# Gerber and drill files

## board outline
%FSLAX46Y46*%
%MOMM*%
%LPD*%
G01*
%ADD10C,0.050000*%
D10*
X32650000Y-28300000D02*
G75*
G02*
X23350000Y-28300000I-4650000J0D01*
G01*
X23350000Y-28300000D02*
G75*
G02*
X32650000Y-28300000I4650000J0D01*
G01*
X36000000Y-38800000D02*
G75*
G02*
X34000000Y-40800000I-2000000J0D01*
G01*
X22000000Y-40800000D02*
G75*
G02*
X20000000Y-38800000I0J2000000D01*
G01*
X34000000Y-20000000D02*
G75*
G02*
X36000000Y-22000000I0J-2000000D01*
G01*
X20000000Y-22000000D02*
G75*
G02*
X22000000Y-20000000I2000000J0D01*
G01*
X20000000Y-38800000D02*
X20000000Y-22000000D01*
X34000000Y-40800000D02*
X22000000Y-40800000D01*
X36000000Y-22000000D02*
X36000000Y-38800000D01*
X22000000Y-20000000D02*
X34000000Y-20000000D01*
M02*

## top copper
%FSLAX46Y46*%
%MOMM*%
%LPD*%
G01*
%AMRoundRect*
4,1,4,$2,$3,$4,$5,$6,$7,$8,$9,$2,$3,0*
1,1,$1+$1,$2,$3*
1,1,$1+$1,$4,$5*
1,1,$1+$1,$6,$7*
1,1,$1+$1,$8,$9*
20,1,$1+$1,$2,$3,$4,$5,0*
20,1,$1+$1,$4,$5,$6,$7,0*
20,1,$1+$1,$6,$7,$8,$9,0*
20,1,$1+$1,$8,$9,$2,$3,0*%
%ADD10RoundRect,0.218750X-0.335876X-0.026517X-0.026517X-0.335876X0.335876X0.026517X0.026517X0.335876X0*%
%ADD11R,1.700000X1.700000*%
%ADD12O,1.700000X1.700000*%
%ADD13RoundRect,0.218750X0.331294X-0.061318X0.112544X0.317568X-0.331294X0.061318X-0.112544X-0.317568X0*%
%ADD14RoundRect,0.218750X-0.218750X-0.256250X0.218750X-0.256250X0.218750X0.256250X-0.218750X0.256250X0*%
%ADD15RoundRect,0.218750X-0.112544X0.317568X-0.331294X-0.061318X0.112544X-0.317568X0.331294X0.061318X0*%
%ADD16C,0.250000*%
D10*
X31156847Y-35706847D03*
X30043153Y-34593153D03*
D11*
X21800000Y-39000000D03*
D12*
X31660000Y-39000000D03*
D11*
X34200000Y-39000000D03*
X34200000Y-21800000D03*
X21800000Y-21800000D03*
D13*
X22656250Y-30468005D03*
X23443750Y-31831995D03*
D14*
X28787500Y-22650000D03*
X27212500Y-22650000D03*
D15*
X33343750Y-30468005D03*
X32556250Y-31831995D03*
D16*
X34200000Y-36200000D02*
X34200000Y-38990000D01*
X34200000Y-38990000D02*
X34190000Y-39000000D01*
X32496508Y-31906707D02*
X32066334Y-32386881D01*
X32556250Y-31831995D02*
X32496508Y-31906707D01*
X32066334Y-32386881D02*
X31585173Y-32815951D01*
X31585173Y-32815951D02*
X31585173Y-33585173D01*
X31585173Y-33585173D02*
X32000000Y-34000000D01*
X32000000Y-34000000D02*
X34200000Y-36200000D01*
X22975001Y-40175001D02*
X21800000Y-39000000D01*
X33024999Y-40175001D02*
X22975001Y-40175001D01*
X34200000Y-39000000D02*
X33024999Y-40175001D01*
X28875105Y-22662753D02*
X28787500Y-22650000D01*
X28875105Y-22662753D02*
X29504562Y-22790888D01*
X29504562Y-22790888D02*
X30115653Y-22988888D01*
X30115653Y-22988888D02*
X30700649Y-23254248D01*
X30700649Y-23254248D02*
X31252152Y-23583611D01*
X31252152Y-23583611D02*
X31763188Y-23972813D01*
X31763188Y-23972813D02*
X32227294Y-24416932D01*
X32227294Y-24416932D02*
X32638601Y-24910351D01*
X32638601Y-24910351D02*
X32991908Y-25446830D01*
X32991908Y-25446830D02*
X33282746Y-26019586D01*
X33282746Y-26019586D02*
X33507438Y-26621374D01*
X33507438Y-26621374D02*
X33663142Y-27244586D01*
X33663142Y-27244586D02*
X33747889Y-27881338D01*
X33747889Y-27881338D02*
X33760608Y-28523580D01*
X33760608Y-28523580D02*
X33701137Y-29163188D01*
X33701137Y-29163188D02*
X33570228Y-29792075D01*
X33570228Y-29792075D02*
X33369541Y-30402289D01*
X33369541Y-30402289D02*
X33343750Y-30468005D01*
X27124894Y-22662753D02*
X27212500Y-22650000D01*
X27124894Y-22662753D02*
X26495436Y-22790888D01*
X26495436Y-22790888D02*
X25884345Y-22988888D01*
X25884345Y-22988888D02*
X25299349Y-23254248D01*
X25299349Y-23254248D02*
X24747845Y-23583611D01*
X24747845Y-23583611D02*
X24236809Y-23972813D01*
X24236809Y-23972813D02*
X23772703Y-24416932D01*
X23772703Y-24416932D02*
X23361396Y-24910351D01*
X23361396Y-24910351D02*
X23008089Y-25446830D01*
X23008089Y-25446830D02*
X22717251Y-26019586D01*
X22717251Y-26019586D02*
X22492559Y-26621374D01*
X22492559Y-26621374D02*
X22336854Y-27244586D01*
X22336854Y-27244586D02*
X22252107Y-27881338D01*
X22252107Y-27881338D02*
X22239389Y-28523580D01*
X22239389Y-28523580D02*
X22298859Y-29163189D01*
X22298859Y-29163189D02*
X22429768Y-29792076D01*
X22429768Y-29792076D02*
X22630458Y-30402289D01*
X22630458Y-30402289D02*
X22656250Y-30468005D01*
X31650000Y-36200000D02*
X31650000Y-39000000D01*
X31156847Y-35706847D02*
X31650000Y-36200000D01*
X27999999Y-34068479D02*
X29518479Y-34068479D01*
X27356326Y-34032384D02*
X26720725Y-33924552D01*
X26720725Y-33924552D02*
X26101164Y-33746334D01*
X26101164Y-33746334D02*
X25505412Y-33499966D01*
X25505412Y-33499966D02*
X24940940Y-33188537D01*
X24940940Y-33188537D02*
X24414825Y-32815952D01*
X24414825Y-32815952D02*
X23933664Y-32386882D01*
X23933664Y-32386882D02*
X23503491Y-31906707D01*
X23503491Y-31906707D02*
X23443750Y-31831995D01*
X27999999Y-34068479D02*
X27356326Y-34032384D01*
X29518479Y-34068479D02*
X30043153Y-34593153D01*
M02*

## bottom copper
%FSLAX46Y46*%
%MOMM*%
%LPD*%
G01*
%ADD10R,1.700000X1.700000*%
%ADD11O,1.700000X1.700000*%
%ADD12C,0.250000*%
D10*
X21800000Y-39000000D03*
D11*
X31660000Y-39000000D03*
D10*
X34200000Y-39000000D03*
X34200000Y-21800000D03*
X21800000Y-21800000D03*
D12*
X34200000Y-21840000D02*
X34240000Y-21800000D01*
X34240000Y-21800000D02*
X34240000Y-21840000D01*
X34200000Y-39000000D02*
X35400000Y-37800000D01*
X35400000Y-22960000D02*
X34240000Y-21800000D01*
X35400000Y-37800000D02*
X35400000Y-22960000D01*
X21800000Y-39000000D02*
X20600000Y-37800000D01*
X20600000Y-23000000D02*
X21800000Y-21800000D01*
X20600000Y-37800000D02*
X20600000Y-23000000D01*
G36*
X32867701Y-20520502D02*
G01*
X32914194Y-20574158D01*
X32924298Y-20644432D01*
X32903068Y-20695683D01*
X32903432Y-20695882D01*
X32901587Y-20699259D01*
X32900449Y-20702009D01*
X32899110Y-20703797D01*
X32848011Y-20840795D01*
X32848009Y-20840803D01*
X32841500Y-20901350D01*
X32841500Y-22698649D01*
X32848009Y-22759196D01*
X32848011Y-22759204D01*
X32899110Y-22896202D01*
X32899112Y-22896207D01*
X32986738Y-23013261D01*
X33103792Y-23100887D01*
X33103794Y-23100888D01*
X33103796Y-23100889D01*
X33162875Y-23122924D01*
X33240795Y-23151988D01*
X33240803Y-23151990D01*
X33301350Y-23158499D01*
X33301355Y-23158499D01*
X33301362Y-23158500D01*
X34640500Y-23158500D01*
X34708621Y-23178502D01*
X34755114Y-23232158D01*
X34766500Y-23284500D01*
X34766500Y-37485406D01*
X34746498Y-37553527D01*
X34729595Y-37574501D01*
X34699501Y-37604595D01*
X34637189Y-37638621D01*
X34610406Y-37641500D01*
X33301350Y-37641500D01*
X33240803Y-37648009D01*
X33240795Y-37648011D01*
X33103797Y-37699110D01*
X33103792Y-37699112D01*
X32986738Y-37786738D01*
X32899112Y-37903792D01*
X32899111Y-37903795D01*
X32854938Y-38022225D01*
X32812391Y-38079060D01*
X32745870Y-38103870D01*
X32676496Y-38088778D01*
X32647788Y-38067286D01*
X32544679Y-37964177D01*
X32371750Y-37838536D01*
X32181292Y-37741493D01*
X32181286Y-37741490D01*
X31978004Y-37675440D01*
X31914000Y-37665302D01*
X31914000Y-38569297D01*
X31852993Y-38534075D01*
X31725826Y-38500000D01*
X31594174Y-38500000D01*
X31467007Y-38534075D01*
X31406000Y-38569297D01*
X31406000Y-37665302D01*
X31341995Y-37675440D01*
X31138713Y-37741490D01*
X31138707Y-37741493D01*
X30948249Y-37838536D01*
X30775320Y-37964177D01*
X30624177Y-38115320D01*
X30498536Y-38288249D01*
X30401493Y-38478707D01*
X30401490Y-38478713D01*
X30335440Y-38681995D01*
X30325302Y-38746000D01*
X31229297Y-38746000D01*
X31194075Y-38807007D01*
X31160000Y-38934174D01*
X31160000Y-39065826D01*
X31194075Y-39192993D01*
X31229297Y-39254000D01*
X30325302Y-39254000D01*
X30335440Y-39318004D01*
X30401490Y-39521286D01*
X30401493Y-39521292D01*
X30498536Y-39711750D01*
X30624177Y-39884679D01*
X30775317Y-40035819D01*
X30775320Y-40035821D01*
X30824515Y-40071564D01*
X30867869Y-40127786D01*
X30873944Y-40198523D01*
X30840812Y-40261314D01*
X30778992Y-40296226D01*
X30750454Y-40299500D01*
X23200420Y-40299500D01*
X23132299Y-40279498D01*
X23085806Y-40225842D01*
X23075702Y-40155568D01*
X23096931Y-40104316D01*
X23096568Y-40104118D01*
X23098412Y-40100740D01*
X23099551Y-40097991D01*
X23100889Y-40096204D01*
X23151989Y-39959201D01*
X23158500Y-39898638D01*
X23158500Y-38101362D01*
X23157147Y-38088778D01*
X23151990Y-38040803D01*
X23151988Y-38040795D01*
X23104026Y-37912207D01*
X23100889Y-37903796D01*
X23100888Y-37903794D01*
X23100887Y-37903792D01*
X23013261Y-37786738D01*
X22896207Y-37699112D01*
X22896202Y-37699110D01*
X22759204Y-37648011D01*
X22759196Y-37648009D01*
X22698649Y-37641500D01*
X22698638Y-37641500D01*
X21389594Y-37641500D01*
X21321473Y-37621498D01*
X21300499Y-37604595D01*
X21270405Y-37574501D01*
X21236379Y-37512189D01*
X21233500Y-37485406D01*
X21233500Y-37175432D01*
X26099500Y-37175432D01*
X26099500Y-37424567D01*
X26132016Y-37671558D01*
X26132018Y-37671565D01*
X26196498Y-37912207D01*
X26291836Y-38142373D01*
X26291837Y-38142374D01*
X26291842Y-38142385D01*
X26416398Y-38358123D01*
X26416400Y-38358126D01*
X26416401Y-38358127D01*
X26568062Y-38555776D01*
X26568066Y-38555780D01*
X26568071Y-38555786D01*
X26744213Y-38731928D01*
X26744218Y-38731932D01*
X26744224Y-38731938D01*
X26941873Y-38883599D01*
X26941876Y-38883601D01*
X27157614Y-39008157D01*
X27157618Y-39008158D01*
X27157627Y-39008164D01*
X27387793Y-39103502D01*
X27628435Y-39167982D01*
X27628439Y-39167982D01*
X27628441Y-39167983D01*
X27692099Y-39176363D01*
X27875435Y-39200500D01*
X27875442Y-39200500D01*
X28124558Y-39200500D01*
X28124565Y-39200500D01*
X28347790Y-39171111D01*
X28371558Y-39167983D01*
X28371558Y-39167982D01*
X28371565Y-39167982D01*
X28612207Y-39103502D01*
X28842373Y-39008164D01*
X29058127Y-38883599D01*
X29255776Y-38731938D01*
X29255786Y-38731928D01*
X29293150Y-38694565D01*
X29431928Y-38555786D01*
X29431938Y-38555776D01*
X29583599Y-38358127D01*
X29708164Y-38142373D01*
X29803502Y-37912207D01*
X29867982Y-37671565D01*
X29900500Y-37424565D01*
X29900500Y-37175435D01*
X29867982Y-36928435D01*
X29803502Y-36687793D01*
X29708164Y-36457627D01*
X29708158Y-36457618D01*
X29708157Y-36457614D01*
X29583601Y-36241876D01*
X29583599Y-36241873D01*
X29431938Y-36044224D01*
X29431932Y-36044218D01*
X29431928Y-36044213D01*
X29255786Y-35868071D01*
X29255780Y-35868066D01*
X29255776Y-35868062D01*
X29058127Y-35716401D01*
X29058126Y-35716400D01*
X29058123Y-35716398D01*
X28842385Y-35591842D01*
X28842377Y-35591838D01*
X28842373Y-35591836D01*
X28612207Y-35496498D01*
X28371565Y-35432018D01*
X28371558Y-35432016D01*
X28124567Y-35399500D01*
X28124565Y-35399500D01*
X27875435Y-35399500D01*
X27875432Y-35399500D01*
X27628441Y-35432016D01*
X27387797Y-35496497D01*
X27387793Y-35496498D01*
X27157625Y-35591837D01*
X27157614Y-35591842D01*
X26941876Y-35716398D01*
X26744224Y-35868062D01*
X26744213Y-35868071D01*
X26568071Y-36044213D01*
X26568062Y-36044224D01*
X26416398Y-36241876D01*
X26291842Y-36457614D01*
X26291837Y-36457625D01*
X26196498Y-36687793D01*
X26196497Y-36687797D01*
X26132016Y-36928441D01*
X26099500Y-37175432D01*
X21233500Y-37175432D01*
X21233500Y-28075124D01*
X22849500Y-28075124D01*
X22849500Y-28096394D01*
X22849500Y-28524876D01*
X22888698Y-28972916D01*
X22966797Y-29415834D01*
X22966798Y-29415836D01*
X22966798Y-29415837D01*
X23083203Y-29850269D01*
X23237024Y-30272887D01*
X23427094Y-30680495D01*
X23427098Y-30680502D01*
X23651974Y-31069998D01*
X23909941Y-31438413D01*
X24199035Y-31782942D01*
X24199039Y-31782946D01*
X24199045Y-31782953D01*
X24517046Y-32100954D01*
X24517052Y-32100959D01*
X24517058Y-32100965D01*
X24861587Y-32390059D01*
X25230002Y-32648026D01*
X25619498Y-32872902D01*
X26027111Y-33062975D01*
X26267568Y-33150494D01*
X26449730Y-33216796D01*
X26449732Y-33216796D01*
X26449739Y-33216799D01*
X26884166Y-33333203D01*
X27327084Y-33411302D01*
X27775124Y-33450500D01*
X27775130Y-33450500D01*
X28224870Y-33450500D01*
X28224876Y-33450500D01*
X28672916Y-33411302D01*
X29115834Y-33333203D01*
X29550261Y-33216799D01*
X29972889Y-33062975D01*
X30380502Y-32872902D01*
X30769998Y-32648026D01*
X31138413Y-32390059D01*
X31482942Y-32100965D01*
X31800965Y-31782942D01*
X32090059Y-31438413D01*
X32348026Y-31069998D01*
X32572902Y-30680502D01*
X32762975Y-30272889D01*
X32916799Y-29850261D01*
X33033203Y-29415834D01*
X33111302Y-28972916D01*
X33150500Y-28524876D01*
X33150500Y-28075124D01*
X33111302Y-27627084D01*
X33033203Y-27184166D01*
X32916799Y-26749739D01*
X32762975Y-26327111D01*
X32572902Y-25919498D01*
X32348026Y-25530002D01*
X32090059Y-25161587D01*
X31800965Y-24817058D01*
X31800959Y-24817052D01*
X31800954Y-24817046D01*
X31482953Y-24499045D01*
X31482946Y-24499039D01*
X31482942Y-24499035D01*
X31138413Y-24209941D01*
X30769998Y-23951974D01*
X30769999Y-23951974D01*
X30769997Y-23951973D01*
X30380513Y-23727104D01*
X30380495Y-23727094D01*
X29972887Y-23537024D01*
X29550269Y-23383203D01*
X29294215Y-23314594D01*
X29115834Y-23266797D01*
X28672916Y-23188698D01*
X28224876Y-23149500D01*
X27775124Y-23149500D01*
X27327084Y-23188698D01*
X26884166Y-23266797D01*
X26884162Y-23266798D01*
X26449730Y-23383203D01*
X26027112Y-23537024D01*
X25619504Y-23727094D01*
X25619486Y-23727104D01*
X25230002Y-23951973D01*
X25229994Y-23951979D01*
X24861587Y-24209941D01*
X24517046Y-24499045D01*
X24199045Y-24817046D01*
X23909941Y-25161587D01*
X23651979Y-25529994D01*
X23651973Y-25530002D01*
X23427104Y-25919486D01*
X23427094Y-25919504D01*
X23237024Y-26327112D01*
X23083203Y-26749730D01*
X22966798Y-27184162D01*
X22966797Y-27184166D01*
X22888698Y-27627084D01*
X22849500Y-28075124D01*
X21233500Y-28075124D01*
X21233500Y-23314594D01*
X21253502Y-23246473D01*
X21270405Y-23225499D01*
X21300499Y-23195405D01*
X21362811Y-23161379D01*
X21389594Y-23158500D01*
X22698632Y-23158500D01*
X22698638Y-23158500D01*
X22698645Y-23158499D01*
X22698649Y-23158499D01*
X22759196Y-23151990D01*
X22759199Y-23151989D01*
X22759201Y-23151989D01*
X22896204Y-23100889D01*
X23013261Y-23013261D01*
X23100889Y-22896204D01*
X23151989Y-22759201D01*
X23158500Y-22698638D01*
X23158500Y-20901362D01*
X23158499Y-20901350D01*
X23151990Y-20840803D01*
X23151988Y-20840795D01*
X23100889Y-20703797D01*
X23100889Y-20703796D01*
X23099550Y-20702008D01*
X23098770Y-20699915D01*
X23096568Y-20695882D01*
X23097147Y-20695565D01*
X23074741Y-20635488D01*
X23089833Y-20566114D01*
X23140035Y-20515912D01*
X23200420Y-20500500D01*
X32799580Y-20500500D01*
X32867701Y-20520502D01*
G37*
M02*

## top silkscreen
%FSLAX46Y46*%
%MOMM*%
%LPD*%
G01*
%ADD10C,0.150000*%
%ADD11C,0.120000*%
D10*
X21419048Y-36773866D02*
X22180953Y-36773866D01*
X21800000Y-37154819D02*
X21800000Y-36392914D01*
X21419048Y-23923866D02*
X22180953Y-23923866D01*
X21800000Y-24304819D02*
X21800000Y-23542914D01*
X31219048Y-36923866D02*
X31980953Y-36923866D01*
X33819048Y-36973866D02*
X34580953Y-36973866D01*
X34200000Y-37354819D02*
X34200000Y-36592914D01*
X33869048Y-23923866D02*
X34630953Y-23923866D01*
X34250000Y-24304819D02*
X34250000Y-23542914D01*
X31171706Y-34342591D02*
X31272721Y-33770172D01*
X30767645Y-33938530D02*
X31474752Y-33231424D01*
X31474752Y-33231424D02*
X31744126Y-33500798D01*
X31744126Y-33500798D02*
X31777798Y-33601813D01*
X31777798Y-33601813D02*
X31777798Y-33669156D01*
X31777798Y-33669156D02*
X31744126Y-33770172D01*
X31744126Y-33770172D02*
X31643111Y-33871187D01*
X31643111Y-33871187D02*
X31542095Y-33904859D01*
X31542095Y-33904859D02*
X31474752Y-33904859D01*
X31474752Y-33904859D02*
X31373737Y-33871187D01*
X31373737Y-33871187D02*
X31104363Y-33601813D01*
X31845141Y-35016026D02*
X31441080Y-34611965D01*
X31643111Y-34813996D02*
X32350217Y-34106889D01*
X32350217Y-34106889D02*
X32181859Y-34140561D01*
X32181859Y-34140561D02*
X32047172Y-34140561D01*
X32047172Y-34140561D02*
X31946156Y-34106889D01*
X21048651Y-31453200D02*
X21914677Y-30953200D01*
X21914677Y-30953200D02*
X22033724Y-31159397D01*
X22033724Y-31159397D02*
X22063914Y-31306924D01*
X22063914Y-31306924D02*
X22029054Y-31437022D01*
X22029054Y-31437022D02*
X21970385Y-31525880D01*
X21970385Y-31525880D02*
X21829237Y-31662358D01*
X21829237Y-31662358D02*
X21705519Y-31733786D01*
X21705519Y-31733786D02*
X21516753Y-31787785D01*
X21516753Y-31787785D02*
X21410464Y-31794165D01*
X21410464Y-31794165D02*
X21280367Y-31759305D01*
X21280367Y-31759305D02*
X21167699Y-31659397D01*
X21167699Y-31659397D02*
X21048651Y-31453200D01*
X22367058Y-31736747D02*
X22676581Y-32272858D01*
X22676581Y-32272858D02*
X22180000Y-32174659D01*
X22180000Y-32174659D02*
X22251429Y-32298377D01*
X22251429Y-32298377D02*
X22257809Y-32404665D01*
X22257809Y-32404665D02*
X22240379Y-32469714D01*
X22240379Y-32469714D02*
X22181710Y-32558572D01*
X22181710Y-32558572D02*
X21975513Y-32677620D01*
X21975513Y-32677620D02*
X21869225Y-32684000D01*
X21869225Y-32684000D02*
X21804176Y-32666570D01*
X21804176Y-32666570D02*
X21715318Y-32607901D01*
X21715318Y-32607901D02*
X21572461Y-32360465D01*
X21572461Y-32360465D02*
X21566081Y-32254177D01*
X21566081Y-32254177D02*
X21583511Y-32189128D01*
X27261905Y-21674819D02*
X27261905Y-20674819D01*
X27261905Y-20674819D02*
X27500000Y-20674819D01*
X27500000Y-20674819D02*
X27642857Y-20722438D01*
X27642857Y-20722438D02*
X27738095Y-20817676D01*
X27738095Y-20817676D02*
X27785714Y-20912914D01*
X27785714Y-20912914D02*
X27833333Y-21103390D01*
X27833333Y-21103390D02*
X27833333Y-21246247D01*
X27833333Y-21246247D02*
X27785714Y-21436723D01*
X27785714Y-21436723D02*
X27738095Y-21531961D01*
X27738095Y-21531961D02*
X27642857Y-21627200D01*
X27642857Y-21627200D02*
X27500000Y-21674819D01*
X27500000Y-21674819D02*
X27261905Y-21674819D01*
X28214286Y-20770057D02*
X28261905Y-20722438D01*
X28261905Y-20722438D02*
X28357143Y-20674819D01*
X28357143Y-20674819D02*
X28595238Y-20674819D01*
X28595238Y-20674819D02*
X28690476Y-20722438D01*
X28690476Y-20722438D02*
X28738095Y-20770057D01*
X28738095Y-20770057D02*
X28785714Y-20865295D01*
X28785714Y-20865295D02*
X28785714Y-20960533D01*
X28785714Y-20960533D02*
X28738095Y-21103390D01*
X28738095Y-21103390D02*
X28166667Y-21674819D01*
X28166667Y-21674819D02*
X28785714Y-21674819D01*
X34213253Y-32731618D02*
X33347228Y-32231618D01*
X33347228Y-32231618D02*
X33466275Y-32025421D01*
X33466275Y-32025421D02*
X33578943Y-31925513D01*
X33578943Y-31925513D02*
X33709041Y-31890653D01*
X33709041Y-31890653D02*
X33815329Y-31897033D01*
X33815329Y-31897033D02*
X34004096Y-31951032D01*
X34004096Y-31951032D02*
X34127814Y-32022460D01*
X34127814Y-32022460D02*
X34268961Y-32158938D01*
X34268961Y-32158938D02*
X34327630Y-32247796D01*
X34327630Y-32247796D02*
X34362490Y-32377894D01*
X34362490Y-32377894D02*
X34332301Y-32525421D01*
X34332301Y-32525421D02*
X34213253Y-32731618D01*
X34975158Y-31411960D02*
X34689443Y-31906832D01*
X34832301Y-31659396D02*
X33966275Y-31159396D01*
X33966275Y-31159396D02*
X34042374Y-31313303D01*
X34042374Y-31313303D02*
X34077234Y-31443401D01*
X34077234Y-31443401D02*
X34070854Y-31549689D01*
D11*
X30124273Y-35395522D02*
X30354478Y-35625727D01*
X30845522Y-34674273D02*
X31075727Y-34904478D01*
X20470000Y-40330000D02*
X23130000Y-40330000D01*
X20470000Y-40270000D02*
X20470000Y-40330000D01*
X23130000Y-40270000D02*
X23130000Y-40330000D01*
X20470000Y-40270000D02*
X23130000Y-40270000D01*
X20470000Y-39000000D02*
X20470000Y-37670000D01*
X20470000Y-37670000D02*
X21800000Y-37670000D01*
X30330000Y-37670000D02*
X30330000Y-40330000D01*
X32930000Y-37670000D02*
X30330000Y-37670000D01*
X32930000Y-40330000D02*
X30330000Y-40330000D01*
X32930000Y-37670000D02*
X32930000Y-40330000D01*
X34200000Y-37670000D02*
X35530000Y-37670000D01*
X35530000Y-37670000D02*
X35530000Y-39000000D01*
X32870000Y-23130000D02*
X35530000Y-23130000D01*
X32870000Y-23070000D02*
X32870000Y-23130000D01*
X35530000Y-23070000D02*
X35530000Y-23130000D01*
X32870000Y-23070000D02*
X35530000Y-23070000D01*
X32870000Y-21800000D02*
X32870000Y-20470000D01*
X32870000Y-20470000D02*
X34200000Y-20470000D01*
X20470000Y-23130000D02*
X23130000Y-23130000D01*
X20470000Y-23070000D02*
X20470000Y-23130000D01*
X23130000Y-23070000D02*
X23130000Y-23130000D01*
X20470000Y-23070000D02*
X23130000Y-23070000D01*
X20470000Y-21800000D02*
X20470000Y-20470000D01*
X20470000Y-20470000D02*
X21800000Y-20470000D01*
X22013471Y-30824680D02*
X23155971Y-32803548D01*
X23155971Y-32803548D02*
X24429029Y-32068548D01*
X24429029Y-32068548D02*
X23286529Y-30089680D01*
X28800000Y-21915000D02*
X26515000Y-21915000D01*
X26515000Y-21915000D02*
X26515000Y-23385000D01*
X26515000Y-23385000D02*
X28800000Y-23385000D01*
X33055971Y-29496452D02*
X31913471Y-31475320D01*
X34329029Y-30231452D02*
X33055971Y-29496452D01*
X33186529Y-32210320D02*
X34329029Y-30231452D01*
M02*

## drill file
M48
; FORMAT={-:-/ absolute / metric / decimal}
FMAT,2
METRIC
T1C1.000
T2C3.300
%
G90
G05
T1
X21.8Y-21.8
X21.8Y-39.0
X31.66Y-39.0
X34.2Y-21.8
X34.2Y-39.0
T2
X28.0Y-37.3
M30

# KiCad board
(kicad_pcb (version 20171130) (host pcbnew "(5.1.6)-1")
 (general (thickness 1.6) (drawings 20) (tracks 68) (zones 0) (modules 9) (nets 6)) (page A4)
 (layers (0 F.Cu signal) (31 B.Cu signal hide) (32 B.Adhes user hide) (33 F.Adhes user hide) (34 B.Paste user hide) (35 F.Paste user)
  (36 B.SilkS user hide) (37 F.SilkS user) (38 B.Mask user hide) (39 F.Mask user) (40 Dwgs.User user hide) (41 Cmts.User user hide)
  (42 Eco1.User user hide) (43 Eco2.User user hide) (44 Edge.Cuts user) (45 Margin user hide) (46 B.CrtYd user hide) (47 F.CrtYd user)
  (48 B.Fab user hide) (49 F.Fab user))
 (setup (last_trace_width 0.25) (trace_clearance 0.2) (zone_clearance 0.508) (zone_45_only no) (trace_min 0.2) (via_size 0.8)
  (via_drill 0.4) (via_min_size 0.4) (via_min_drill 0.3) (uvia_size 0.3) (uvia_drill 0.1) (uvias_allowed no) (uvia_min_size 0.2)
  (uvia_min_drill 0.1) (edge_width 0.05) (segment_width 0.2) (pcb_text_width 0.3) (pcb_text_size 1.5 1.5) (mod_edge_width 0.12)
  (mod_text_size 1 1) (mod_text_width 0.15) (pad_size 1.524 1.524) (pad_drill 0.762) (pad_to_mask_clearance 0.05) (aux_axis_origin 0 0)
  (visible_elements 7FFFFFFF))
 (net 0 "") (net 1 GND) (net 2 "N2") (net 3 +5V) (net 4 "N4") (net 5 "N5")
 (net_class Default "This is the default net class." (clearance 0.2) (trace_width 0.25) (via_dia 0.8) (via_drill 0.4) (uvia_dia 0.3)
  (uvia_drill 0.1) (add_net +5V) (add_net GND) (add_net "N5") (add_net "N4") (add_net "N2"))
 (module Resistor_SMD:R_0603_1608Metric (layer F.Cu) (at 30.6 35.15 315)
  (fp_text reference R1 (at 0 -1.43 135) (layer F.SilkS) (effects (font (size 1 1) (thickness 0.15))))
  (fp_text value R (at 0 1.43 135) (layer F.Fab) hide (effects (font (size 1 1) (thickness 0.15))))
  (fp_line (start -0.162779 0.51) (end 0.162779 0.51) (layer F.SilkS) (width 0.12))
  (fp_line (start -0.162779 -0.51) (end 0.162779 -0.51) (layer F.SilkS) (width 0.12))
  (pad 2 smd roundrect (at 0.7875 0 315) (size 0.875 0.95) (layers F.Cu F.Paste F.Mask) (roundrect_rratio 0.25) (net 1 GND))
  (pad 1 smd roundrect (at -0.7875 0 315) (size 0.875 0.95) (layers F.Cu F.Paste F.Mask) (roundrect_rratio 0.25) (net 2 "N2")))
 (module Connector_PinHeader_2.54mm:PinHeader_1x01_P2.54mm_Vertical (layer F.Cu) (at 21.8 39)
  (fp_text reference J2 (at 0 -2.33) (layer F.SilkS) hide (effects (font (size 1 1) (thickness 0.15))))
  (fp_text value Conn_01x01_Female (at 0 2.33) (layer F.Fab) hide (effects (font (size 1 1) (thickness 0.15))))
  (fp_line (start -1.33 1.33) (end 1.33 1.33) (layer F.SilkS) (width 0.12))
  (fp_line (start -1.33 1.27) (end -1.33 1.33) (layer F.SilkS) (width 0.12))
  (fp_line (start 1.33 1.27) (end 1.33 1.33) (layer F.SilkS) (width 0.12))
  (fp_line (start -1.33 1.27) (end 1.33 1.27) (layer F.SilkS) (width 0.12))
  (fp_line (start -1.33 0) (end -1.33 -1.33) (layer F.SilkS) (width 0.12))
  (fp_line (start -1.33 -1.33) (end 0 -1.33) (layer F.SilkS) (width 0.12))
  (pad 1 thru_hole rect (at 0 0) (size 1.7 1.7) (drill 1) (layers *.Cu *.Mask) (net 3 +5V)))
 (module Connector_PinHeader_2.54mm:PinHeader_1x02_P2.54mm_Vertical (layer F.Cu) (at 34.2 39 270)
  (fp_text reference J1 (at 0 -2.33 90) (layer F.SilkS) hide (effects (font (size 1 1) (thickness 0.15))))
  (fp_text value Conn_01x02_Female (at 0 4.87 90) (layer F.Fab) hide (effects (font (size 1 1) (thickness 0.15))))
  (fp_line (start -1.33 3.87) (end 1.33 3.87) (layer F.SilkS) (width 0.12))
  (fp_line (start -1.33 1.27) (end -1.33 3.87) (layer F.SilkS) (width 0.12))
  (fp_line (start 1.33 1.27) (end 1.33 3.87) (layer F.SilkS) (width 0.12))
  (fp_line (start -1.33 1.27) (end 1.33 1.27) (layer F.SilkS) (width 0.12))
  (fp_line (start -1.33 0) (end -1.33 -1.33) (layer F.SilkS) (width 0.12))
  (fp_line (start -1.33 -1.33) (end 0 -1.33) (layer F.SilkS) (width 0.12))
  (pad 2 thru_hole oval (at 0 2.54 270) (size 1.7 1.7) (drill 1) (layers *.Cu *.Mask) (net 1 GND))
  (pad 1 thru_hole rect (at 0 0 270) (size 1.7 1.7) (drill 1) (layers *.Cu *.Mask) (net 3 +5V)))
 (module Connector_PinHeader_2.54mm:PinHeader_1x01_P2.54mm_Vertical (layer F.Cu) (at 34.2 21.8)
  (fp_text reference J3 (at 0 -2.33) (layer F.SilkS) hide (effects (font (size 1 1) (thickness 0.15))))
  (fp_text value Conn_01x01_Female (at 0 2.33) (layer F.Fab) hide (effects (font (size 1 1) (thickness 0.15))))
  (fp_line (start -1.33 1.33) (end 1.33 1.33) (layer F.SilkS) (width 0.12))
  (fp_line (start -1.33 1.27) (end -1.33 1.33) (layer F.SilkS) (width 0.12))
  (fp_line (start 1.33 1.27) (end 1.33 1.33) (layer F.SilkS) (width 0.12))
  (fp_line (start -1.33 1.27) (end 1.33 1.27) (layer F.SilkS) (width 0.12))
  (fp_line (start -1.33 0) (end -1.33 -1.33) (layer F.SilkS) (width 0.12))
  (fp_line (start -1.33 -1.33) (end 0 -1.33) (layer F.SilkS) (width 0.12))
  (pad 1 thru_hole rect (at 0 0) (size 1.7 1.7) (drill 1) (layers *.Cu *.Mask) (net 3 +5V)))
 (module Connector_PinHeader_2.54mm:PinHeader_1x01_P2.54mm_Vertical (layer F.Cu) (at 21.8 21.8)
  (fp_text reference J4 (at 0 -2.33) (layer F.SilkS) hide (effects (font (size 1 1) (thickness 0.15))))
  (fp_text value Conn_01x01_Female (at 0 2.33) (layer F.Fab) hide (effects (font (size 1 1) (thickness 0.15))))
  (fp_line (start -1.33 1.33) (end 1.33 1.33) (layer F.SilkS) (width 0.12))
  (fp_line (start -1.33 1.27) (end -1.33 1.33) (layer F.SilkS) (width 0.12))
  (fp_line (start 1.33 1.27) (end 1.33 1.33) (layer F.SilkS) (width 0.12))
  (fp_line (start -1.33 1.27) (end 1.33 1.27) (layer F.SilkS) (width 0.12))
  (fp_line (start -1.33 0) (end -1.33 -1.33) (layer F.SilkS) (width 0.12))
  (fp_line (start -1.33 -1.33) (end 0 -1.33) (layer F.SilkS) (width 0.12))
  (pad 1 thru_hole rect (at 0 0) (size 1.7 1.7) (drill 1) (layers *.Cu *.Mask) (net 3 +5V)))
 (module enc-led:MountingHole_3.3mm (layer F.Cu) (at 28 37.3)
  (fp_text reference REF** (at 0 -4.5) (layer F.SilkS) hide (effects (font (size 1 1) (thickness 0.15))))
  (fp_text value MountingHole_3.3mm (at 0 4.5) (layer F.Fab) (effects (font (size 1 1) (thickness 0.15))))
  (pad "" np_thru_hole circle (at 0 0) (size 3.3 3.3) (drill 3.3) (layers *.Cu *.Mask)))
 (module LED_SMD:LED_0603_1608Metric (layer F.Cu) (at 23.05 31.15 120)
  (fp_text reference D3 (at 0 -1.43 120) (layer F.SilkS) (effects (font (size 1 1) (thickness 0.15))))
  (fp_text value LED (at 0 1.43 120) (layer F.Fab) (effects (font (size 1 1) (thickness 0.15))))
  (fp_line (start 0.8 -0.735) (end -1.485 -0.735) (layer F.SilkS) (width 0.12))
  (fp_line (start -1.485 -0.735) (end -1.485 0.735) (layer F.SilkS) (width 0.12))
  (fp_line (start -1.485 0.735) (end 0.8 0.735) (layer F.SilkS) (width 0.12))
  (pad 2 smd roundrect (at 0.7875 0 120) (size 0.875 0.95) (layers F.Cu F.Paste F.Mask) (roundrect_rratio 0.25) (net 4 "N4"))
  (pad 1 smd roundrect (at -0.7875 0 120) (size 0.875 0.95) (layers F.Cu F.Paste F.Mask) (roundrect_rratio 0.25) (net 2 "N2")))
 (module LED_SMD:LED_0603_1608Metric (layer F.Cu) (at 28 22.65)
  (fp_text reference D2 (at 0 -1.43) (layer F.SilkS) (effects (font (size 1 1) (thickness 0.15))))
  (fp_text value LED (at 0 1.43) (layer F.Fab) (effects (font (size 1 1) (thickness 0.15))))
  (fp_line (start 0.8 -0.735) (end -1.485 -0.735) (layer F.SilkS) (width 0.12))
  (fp_line (start -1.485 -0.735) (end -1.485 0.735) (layer F.SilkS) (width 0.12))
  (fp_line (start -1.485 0.735) (end 0.8 0.735) (layer F.SilkS) (width 0.12))
  (pad 2 smd roundrect (at 0.7875 0) (size 0.875 0.95) (layers F.Cu F.Paste F.Mask) (roundrect_rratio 0.25) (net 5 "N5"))
  (pad 1 smd roundrect (at -0.7875 0) (size 0.875 0.95) (layers F.Cu F.Paste F.Mask) (roundrect_rratio 0.25) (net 4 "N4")))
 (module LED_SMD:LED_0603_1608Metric (layer F.Cu) (at 32.95 31.15 240)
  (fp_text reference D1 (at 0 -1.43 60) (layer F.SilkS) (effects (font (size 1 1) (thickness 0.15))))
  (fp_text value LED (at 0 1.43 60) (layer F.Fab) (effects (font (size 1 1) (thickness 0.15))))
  (fp_line (start -1.485 0.735) (end 0.8 0.735) (layer F.SilkS) (width 0.12))
  (fp_line (start -1.485 -0.735) (end -1.485 0.735) (layer F.SilkS) (width 0.12))
  (fp_line (start 0.8 -0.735) (end -1.485 -0.735) (layer F.SilkS) (width 0.12))
  (pad 1 smd roundrect (at -0.7875 0 240) (size 0.875 0.95) (layers F.Cu F.Paste F.Mask) (roundrect_rratio 0.25) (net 5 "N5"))
  (pad 2 smd roundrect (at 0.7875 0 240) (size 0.875 0.95) (layers F.Cu F.Paste F.Mask) (roundrect_rratio 0.25) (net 3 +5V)))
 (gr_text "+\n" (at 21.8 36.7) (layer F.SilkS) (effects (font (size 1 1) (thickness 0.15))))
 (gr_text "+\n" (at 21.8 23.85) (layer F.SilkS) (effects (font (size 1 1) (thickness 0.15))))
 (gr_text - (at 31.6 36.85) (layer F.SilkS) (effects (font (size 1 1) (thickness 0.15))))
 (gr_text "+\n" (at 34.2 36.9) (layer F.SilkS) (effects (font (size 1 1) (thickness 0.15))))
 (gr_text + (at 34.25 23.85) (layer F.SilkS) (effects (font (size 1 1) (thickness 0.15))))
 (gr_circle (center 28 28.3) (end 32.65 28.3) (layer Edge.Cuts) (width 0.05))
 (gr_arc (start 34 38.8) (end 34 40.8) (angle -90) (layer Edge.Cuts) (width 0.05))
 (gr_arc (start 22 38.8) (end 20 38.8) (angle -90) (layer Edge.Cuts) (width 0.05))
 (gr_arc (start 34 22) (end 36 22) (angle -90) (layer Edge.Cuts) (width 0.05))
 (gr_arc (start 22 22) (end 22 20) (angle -90) (layer Edge.Cuts) (width 0.05))
 (gr_line (start 20 38.8) (end 20 22) (layer Edge.Cuts) (width 0.05))
 (gr_line (start 34 40.8) (end 22 40.8) (layer Edge.Cuts) (width 0.05))
 (gr_line (start 36 22) (end 36 38.8) (layer Edge.Cuts) (width 0.05))
 (gr_line (start 22 20) (end 34 20) (layer Edge.Cuts) (width 0.05))
 (segment (start 34.2 36.2) (end 34.2 38.99) (width 0.25) (layer F.Cu) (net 3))
 (segment (start 34.2 38.99) (end 34.19 39) (width 0.25) (layer F.Cu) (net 3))
 (segment (start 32.496508 31.906707) (end 32.066334 32.386881) (width 0.25) (layer F.Cu) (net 3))
 (segment (start 32.55625 31.831995) (end 32.496508 31.906707) (width 0.25) (layer F.Cu) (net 3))
 (segment (start 32.066334 32.386881) (end 31.585173 32.815951) (width 0.25) (layer F.Cu) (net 3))
 (segment (start 31.585173 32.815951) (end 31.585173 33.585173) (width 0.25) (layer F.Cu) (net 3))
 (segment (start 31.585173 33.585173) (end 32 34) (width 0.25) (layer F.Cu) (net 3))
 (segment (start 32 34) (end 34.2 36.2) (width 0.25) (layer F.Cu) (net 3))
 (segment (start 22.975001 40.175001) (end 21.8 39) (width 0.25) (layer F.Cu) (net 3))
 (segment (start 33.024999 40.175001) (end 22.975001 40.175001) (width 0.25) (layer F.Cu) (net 3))
 (segment (start 34.2 39) (end 33.024999 40.175001) (width 0.25) (layer F.Cu) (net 3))
 (segment (start 34.2 21.84) (end 34.24 21.8) (width 0.25) (layer B.Cu) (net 3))
 (segment (start 34.24 21.8) (end 34.24 21.84) (width 0.25) (layer B.Cu) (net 3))
 (segment (start 34.2 39) (end 35.4 37.8) (width 0.25) (layer B.Cu) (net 3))
 (segment (start 35.4 22.96) (end 34.24 21.8) (width 0.25) (layer B.Cu) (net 3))
 (segment (start 35.4 37.8) (end 35.4 22.96) (width 0.25) (layer B.Cu) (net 3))
 (segment (start 21.8 39) (end 20.6 37.8) (width 0.25) (layer B.Cu) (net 3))
 (segment (start 20.6 23) (end 21.8 21.8) (width 0.25) (layer B.Cu) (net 3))
 (segment (start 20.6 37.8) (end 20.6 23) (width 0.25) (layer B.Cu) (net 3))
 (segment (start 28.875105 22.662753) (end 28.7875 22.65) (width 0.25) (layer F.Cu) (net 5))
 (segment (start 28.875105 22.662753) (end 29.504562 22.790888) (width 0.25) (layer F.Cu) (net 5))
 (segment (start 29.504562 22.790888) (end 30.115653 22.988888) (width 0.25) (layer F.Cu) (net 5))
 (segment (start 30.115653 22.988888) (end 30.700649 23.254248) (width 0.25) (layer F.Cu) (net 5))
 (segment (start 30.700649 23.254248) (end 31.252152 23.583611) (width 0.25) (layer F.Cu) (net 5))
 (segment (start 31.252152 23.583611) (end 31.763188 23.972813) (width 0.25) (layer F.Cu) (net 5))
 (segment (start 31.763188 23.972813) (end 32.227294 24.416932) (width 0.25) (layer F.Cu) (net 5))
 (segment (start 32.227294 24.416932) (end 32.638601 24.910351) (width 0.25) (layer F.Cu) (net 5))
 (segment (start 32.638601 24.910351) (end 32.991908 25.44683) (width 0.25) (layer F.Cu) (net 5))
 (segment (start 32.991908 25.44683) (end 33.282746 26.019586) (width 0.25) (layer F.Cu) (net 5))
 (segment (start 33.282746 26.019586) (end 33.507438 26.621374) (width 0.25) (layer F.Cu) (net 5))
 (segment (start 33.507438 26.621374) (end 33.663142 27.244586) (width 0.25) (layer F.Cu) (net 5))
 (segment (start 33.663142 27.244586) (end 33.747889 27.881338) (width 0.25) (layer F.Cu) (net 5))
 (segment (start 33.747889 27.881338) (end 33.760608 28.52358) (width 0.25) (layer F.Cu) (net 5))
 (segment (start 33.760608 28.52358) (end 33.701137 29.163188) (width 0.25) (layer F.Cu) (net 5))
 (segment (start 33.701137 29.163188) (end 33.570228 29.792075) (width 0.25) (layer F.Cu) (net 5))
 (segment (start 33.570228 29.792075) (end 33.369541 30.402289) (width 0.25) (layer F.Cu) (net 5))
 (segment (start 33.369541 30.402289) (end 33.34375 30.468005) (width 0.25) (layer F.Cu) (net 5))
 (segment (start 27.124894 22.662753) (end 27.2125 22.65) (width 0.25) (layer F.Cu) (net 4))
 (segment (start 27.124894 22.662753) (end 26.495436 22.790888) (width 0.25) (layer F.Cu) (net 4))
 (segment (start 26.495436 22.790888) (end 25.884345 22.988888) (width 0.25) (layer F.Cu) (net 4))
 (segment (start 25.884345 22.988888) (end 25.299349 23.254248) (width 0.25) (layer F.Cu) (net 4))
 (segment (start 25.299349 23.254248) (end 24.747845 23.583611) (width 0.25) (layer F.Cu) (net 4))
 (segment (start 24.747845 23.583611) (end 24.236809 23.972813) (width 0.25) (layer F.Cu) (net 4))
 (segment (start 24.236809 23.972813) (end 23.772703 24.416932) (width 0.25) (layer F.Cu) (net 4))
 (segment (start 23.772703 24.416932) (end 23.361396 24.910351) (width 0.25) (layer F.Cu) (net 4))
 (segment (start 23.361396 24.910351) (end 23.008089 25.44683) (width 0.25) (layer F.Cu) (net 4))
 (segment (start 23.008089 25.44683) (end 22.717251 26.019586) (width 0.25) (layer F.Cu) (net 4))
 (segment (start 22.717251 26.019586) (end 22.492559 26.621374) (width 0.25) (layer F.Cu) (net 4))
 (segment (start 22.492559 26.621374) (end 22.336854 27.244586) (width 0.25) (layer F.Cu) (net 4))
 (segment (start 22.336854 27.244586) (end 22.252107 27.881338) (width 0.25) (layer F.Cu) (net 4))
 (segment (start 22.252107 27.881338) (end 22.239389 28.52358) (width 0.25) (layer F.Cu) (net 4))
 (segment (start 22.239389 28.52358) (end 22.298859 29.163189) (width 0.25) (layer F.Cu) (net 4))
 (segment (start 22.298859 29.163189) (end 22.429768 29.792076) (width 0.25) (layer F.Cu) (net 4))
 (segment (start 22.429768 29.792076) (end 22.630458 30.402289) (width 0.25) (layer F.Cu) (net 4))
 (segment (start 22.630458 30.402289) (end 22.65625 30.468005) (width 0.25) (layer F.Cu) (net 4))
 (segment (start 31.65 36.2) (end 31.65 39) (width 0.25) (layer F.Cu) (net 1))
 (segment (start 31.156847 35.706847) (end 31.65 36.2) (width 0.25) (layer F.Cu) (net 1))
 (segment (start 27.999999 34.068479) (end 29.518479 34.068479) (width 0.25) (layer F.Cu) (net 2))
 (segment (start 27.356326 34.032384) (end 26.720725 33.924552) (width 0.25) (layer F.Cu) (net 2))
 (segment (start 26.720725 33.924552) (end 26.101164 33.746334) (width 0.25) (layer F.Cu) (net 2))
 (segment (start 26.101164 33.746334) (end 25.505412 33.499966) (width 0.25) (layer F.Cu) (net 2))
 (segment (start 25.505412 33.499966) (end 24.94094 33.188537) (width 0.25) (layer F.Cu) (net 2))
 (segment (start 24.94094 33.188537) (end 24.414825 32.815952) (width 0.25) (layer F.Cu) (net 2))
 (segment (start 24.414825 32.815952) (end 23.933664 32.386882) (width 0.25) (layer F.Cu) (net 2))
 (segment (start 23.933664 32.386882) (end 23.503491 31.906707) (width 0.25) (layer F.Cu) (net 2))
 (segment (start 23.503491 31.906707) (end 23.44375 31.831995) (width 0.25) (layer F.Cu) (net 2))
 (segment (start 27.999999 34.068479) (end 27.356326 34.032384) (width 0.25) (layer F.Cu) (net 2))
 (segment (start 29.518479 34.068479) (end 30.043153 34.593153) (width 0.25) (layer F.Cu) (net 2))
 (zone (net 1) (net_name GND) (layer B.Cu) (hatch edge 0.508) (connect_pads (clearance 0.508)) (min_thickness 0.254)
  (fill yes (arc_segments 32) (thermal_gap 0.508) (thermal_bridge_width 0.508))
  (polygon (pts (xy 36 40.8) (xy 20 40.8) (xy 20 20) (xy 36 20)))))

